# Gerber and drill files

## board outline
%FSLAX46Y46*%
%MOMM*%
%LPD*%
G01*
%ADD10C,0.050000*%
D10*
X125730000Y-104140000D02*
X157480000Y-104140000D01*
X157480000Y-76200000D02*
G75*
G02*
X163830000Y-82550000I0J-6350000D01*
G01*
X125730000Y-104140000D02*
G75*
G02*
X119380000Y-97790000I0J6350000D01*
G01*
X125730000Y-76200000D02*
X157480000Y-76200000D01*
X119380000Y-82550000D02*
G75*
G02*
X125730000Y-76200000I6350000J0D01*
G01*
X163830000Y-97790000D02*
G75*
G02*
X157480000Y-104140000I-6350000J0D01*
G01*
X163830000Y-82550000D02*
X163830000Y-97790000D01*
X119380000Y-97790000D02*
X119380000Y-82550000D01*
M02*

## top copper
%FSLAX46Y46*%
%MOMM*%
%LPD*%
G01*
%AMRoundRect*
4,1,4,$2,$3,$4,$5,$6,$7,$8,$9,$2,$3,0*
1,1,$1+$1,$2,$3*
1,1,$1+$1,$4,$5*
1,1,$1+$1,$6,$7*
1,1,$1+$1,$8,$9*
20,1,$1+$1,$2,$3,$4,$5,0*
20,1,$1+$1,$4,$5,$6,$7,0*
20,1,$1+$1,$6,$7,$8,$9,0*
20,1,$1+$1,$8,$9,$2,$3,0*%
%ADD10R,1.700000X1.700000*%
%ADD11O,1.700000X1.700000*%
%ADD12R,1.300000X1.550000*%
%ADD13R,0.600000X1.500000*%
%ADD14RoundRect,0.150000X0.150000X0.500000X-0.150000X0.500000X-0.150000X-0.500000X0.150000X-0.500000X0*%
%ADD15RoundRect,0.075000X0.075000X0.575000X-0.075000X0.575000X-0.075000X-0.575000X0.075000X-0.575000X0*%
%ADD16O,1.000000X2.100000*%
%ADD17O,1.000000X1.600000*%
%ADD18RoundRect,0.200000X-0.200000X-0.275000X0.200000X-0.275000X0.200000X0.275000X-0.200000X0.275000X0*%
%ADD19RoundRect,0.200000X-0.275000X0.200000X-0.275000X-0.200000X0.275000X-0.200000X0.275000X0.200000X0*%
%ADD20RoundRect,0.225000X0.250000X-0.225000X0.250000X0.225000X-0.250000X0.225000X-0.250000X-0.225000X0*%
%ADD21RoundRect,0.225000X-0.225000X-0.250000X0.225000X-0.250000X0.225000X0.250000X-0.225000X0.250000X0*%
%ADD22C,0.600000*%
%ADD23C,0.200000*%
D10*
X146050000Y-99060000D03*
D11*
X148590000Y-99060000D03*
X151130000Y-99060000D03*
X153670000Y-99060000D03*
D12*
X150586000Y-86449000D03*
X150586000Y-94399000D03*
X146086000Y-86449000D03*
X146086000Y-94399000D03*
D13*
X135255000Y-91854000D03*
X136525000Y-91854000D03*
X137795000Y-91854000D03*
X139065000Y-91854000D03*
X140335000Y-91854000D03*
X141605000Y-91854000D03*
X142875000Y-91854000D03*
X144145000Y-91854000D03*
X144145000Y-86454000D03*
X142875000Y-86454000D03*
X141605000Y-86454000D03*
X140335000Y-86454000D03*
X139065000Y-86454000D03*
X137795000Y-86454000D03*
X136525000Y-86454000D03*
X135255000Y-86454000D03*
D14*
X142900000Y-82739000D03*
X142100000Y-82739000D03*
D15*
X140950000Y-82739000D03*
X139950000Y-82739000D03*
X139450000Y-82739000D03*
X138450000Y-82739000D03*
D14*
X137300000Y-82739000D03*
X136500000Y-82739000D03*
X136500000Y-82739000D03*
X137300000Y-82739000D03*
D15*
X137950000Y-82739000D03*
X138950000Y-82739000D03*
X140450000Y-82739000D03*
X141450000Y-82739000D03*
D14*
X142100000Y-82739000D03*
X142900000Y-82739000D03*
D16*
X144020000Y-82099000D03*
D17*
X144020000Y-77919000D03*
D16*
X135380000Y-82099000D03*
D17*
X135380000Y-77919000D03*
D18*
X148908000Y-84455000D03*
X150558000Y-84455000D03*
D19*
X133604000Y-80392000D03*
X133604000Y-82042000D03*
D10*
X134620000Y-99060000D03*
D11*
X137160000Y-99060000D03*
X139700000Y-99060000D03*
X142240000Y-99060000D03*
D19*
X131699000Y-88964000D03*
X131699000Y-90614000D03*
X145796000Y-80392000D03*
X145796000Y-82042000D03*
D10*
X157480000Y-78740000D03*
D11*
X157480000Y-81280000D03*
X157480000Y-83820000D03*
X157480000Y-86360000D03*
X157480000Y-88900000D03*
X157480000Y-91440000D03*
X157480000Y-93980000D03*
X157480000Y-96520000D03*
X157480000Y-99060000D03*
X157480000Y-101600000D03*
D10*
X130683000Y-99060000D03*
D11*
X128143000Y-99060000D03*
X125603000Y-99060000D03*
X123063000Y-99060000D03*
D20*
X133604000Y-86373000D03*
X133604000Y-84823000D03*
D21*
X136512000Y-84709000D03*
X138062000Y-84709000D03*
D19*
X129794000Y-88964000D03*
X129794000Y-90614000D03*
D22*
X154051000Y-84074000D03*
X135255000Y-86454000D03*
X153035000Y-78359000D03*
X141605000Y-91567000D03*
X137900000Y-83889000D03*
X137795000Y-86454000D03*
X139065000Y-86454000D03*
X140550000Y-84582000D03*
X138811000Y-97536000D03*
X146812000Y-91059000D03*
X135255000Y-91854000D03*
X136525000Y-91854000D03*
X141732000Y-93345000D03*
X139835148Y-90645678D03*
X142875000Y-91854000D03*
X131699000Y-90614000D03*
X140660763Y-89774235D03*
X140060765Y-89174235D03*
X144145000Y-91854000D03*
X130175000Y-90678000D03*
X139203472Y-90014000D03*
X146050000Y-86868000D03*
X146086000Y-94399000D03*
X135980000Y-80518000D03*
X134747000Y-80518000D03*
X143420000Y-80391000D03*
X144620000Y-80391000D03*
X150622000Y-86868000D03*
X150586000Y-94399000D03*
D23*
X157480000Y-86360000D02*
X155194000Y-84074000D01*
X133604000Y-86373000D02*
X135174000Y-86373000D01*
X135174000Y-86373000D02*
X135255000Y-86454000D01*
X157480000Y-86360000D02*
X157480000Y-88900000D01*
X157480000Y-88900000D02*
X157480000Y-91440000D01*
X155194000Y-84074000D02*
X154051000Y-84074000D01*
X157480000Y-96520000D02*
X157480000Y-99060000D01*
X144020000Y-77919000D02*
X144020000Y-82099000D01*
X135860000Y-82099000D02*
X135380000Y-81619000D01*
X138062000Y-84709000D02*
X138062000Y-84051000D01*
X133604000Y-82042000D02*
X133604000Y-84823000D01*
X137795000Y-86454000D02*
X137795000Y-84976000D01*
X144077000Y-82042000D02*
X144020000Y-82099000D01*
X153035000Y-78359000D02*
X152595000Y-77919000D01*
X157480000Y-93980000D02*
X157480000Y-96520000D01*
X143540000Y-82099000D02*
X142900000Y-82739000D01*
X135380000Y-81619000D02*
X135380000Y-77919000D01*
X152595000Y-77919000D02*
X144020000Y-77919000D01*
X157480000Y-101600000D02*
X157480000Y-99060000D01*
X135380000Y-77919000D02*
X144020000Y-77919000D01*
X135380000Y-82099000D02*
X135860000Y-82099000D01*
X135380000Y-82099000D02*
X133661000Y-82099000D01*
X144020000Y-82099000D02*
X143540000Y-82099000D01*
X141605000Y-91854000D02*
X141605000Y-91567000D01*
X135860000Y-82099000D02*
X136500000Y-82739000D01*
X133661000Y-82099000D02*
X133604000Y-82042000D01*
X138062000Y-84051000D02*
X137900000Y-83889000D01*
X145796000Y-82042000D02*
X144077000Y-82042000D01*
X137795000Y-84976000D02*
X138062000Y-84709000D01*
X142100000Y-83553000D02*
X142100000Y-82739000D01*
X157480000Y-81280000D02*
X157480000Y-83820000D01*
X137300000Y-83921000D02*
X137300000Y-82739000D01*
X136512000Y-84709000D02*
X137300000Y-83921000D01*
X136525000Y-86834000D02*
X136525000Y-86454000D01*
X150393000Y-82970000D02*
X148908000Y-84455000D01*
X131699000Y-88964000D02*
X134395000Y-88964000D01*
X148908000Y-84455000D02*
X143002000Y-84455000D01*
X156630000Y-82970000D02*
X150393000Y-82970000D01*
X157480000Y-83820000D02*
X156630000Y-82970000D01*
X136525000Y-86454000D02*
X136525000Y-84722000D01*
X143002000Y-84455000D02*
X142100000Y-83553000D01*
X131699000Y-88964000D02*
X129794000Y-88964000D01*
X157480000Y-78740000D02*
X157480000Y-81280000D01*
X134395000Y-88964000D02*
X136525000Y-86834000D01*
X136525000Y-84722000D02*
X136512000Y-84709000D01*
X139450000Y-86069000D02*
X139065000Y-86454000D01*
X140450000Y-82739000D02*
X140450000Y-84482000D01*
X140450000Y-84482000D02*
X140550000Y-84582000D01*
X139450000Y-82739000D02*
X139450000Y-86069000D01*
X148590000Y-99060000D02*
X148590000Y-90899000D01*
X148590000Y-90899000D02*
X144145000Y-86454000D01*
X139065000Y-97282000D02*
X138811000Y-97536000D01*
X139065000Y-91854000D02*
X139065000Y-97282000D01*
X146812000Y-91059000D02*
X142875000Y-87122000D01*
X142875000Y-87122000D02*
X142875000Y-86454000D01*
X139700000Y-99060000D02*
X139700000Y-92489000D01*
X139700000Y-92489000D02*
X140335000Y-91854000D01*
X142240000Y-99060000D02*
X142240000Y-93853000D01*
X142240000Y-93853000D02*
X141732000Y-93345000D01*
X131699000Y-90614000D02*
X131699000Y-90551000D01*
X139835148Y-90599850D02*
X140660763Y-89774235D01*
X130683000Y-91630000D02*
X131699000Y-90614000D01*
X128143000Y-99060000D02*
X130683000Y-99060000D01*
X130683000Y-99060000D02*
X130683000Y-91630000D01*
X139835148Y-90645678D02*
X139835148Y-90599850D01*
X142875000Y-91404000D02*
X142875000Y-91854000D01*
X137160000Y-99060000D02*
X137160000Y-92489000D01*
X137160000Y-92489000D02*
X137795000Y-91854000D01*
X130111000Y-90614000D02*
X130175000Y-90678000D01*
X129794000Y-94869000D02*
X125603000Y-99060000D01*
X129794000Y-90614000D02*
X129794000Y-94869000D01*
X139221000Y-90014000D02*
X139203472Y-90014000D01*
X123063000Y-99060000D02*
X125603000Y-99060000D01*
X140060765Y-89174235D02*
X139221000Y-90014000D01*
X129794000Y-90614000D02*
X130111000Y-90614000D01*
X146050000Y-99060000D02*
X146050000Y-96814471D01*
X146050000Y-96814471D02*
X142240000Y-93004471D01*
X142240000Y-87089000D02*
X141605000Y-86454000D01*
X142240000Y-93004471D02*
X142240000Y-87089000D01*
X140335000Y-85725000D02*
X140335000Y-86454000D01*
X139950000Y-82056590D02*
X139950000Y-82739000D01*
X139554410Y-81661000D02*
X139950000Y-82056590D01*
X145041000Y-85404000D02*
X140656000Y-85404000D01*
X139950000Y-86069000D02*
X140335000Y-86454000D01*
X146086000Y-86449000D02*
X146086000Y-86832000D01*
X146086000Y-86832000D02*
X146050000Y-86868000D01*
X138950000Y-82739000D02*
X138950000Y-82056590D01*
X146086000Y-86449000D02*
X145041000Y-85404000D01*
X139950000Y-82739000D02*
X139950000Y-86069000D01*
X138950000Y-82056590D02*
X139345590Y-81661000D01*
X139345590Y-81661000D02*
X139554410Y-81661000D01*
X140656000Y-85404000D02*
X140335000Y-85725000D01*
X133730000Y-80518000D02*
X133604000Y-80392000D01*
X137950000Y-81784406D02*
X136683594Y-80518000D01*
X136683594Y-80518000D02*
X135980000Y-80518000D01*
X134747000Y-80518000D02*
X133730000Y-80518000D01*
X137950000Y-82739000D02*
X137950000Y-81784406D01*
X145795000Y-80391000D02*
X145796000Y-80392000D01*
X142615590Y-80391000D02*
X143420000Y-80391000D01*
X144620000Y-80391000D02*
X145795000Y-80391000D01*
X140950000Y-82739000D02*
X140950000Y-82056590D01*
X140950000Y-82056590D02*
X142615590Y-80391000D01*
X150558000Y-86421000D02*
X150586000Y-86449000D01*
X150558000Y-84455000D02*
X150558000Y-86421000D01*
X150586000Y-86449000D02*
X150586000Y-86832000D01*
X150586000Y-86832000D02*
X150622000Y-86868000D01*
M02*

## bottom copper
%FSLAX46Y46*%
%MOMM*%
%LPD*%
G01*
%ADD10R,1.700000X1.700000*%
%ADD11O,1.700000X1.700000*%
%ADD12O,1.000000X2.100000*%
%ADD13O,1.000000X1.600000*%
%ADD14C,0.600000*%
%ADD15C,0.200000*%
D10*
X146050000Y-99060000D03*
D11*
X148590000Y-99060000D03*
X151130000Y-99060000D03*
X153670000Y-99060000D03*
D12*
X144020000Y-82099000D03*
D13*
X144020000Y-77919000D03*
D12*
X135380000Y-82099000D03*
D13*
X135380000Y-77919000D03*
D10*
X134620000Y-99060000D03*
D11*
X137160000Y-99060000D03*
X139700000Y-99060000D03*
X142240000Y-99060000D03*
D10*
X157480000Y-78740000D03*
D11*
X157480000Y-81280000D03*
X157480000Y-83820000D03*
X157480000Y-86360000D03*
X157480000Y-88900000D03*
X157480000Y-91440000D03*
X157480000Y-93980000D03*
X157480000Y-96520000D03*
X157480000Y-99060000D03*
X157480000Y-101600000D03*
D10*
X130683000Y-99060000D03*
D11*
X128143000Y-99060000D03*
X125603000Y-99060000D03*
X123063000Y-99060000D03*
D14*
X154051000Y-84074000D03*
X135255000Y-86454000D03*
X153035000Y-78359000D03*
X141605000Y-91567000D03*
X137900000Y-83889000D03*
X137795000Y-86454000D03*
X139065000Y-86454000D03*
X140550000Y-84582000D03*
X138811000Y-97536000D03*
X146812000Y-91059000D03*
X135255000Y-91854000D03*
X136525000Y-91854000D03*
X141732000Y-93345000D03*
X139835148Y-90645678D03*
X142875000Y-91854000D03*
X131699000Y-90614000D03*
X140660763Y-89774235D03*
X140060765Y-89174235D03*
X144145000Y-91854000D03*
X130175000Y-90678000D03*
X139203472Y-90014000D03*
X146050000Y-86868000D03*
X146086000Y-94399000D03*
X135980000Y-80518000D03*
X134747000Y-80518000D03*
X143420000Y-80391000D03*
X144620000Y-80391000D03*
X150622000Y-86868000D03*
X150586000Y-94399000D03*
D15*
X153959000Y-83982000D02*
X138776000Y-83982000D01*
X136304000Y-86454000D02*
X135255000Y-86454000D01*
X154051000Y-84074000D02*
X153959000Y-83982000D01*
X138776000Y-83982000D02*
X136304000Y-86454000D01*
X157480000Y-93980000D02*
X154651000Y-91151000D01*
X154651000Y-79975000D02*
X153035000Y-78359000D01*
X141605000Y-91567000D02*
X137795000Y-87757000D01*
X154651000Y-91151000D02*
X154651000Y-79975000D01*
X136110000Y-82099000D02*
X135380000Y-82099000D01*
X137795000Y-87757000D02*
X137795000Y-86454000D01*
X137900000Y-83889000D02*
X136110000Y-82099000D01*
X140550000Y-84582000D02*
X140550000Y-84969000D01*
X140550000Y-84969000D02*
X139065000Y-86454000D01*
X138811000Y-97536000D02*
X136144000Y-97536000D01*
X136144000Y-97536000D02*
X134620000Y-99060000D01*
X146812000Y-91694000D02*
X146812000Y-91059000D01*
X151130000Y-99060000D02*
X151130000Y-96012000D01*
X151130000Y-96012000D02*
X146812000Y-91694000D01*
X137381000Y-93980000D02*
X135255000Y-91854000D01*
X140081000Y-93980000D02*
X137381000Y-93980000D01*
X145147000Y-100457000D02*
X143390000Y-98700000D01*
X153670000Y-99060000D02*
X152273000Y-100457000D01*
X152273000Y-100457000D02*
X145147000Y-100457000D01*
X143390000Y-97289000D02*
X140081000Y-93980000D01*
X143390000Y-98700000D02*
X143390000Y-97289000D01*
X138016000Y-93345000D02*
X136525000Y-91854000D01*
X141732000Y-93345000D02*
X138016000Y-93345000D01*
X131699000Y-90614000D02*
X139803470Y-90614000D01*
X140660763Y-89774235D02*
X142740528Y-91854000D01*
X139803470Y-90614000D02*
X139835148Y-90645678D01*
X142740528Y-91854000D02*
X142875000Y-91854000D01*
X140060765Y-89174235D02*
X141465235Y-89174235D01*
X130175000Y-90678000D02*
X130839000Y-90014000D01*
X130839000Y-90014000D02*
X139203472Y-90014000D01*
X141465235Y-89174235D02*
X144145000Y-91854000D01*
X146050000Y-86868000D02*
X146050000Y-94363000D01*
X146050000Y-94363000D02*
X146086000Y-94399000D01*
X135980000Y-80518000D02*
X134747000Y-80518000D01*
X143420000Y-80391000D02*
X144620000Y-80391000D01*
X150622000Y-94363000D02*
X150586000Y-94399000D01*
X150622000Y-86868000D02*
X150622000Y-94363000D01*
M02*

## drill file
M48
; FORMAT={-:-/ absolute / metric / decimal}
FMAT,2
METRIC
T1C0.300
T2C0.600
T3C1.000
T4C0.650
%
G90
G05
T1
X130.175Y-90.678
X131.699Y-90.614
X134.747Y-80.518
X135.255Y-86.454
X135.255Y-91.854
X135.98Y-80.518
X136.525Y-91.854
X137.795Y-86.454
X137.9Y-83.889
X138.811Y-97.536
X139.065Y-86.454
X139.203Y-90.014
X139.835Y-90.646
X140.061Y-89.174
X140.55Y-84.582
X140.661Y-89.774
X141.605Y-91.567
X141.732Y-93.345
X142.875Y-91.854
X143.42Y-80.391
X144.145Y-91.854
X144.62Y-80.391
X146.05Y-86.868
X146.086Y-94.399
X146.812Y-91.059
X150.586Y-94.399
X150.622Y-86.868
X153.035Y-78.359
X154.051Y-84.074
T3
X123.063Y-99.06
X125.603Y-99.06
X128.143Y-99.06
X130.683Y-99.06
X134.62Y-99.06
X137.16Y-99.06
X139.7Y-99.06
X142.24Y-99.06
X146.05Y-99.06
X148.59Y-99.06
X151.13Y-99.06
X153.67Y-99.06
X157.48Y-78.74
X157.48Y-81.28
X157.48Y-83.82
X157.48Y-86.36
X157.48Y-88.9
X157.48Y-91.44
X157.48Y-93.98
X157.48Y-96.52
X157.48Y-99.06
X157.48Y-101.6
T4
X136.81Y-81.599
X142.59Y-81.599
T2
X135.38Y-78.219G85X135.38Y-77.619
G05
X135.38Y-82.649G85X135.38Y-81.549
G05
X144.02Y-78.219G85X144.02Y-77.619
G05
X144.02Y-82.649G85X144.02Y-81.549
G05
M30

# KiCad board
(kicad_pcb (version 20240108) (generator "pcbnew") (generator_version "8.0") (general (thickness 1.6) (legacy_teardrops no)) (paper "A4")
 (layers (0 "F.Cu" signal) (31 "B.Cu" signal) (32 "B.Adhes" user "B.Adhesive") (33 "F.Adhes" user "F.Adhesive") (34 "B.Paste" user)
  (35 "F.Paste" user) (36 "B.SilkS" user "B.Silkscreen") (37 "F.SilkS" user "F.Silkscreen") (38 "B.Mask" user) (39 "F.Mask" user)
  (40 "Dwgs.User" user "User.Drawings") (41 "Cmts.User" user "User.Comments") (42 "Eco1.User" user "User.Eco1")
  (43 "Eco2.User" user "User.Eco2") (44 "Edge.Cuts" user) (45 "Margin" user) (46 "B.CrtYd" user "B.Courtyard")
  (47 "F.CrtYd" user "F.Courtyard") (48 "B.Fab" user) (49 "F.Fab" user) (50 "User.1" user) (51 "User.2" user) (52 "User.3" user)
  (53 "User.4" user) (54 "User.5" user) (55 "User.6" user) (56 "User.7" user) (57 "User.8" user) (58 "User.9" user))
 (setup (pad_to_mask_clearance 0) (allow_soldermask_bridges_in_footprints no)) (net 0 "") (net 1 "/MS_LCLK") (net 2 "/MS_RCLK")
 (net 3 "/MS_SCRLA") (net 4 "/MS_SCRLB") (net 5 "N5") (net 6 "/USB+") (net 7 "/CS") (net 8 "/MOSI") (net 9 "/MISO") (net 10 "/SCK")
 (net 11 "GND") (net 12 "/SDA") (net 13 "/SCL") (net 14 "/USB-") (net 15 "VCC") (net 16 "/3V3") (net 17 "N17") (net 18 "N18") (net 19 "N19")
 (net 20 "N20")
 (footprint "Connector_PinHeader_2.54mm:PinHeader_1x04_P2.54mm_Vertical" (layer "F.Cu") (at 146.05 99.06 90)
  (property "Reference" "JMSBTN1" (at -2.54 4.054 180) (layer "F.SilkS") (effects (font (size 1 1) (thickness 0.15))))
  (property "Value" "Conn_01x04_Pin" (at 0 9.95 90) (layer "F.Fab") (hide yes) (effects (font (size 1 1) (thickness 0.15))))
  (pad "1" thru_hole rect (at 0 0 90) (size 1.7 1.7) (drill 1) (layers "*.Cu" "*.Mask") (remove_unused_layers no) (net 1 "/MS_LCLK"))
  (pad "2" thru_hole oval (at 0 2.54 90) (size 1.7 1.7) (drill 1) (layers "*.Cu" "*.Mask") (remove_unused_layers no) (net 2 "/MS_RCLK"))
  (pad "3" thru_hole oval (at 0 5.08 90) (size 1.7 1.7) (drill 1) (layers "*.Cu" "*.Mask") (remove_unused_layers no) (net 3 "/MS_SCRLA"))
  (pad "4" thru_hole oval (at 0 7.62 90) (size 1.7 1.7) (drill 1) (layers "*.Cu" "*.Mask") (remove_unused_layers no) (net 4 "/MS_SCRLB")))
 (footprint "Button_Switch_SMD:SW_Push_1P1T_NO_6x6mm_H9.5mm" (layer "F.Cu") (at 148.336 90.424 -90)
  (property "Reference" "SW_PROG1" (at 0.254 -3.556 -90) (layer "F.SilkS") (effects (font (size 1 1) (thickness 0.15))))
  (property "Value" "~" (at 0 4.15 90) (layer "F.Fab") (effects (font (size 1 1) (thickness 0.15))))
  (pad "1" smd rect (at -3.975 -2.25 270) (size 1.55 1.3) (layers "F.Cu" "F.Paste" "F.Mask") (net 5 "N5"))
  (pad "1" smd rect (at 3.975 -2.25 270) (size 1.55 1.3) (layers "F.Cu" "F.Paste" "F.Mask") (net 5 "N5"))
  (pad "2" smd rect (at -3.975 2.25 270) (size 1.55 1.3) (layers "F.Cu" "F.Paste" "F.Mask") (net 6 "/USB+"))
  (pad "2" smd rect (at 3.975 2.25 270) (size 1.55 1.3) (layers "F.Cu" "F.Paste" "F.Mask") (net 6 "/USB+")))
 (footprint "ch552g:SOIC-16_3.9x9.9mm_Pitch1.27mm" (layer "F.Cu") (at 139.7 89.154 90)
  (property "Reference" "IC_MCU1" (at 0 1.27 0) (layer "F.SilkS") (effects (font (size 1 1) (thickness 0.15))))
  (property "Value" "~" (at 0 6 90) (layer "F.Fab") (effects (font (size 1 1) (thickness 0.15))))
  (pad "1" smd rect (at -2.7 -4.445 90) (size 1.5 0.6) (layers "F.Cu" "F.Paste" "F.Mask") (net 4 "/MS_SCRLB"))
  (pad "2" smd rect (at -2.7 -3.175 90) (size 1.5 0.6) (layers "F.Cu" "F.Paste" "F.Mask") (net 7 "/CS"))
  (pad "3" smd rect (at -2.7 -1.905 90) (size 1.5 0.6) (layers "F.Cu" "F.Paste" "F.Mask") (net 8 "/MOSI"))
  (pad "4" smd rect (at -2.7 -0.635 90) (size 1.5 0.6) (layers "F.Cu" "F.Paste" "F.Mask") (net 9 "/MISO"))
  (pad "5" smd rect (at -2.7 0.635 90) (size 1.5 0.6) (layers "F.Cu" "F.Paste" "F.Mask") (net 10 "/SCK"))
  (pad "6" smd rect (at -2.7 1.905 90) (size 1.5 0.6) (layers "F.Cu" "F.Paste" "F.Mask") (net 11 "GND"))
  (pad "7" smd rect (at -2.7 3.175 90) (size 1.5 0.6) (layers "F.Cu" "F.Paste" "F.Mask") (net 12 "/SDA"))
  (pad "8" smd rect (at -2.7 4.445 90) (size 1.5 0.6) (layers "F.Cu" "F.Paste" "F.Mask") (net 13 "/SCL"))
  (pad "9" smd rect (at 2.7 4.445 90) (size 1.5 0.6) (layers "F.Cu" "F.Paste" "F.Mask") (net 2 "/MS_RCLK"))
  (pad "10" smd rect (at 2.7 3.175 90) (size 1.5 0.6) (layers "F.Cu" "F.Paste" "F.Mask") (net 3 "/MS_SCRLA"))
  (pad "11" smd rect (at 2.7 1.905 90) (size 1.5 0.6) (layers "F.Cu" "F.Paste" "F.Mask") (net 1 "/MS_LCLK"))
  (pad "12" smd rect (at 2.7 0.635 90) (size 1.5 0.6) (layers "F.Cu" "F.Paste" "F.Mask") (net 6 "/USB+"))
  (pad "13" smd rect (at 2.7 -0.635 90) (size 1.5 0.6) (layers "F.Cu" "F.Paste" "F.Mask") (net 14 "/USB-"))
  (pad "14" smd rect (at 2.7 -1.905 90) (size 1.5 0.6) (layers "F.Cu" "F.Paste" "F.Mask") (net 11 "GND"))
  (pad "15" smd rect (at 2.7 -3.175 90) (size 1.5 0.6) (layers "F.Cu" "F.Paste" "F.Mask") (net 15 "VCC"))
  (pad "16" smd rect (at 2.7 -4.445 90) (size 1.5 0.6) (layers "F.Cu" "F.Paste" "F.Mask") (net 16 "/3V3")))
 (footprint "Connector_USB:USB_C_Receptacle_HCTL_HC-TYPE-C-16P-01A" (layer "F.Cu") (at 139.7 78.994 180)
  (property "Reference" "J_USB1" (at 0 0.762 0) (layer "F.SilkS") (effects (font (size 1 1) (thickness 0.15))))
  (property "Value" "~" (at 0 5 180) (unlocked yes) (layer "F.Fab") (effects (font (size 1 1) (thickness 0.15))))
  (pad "" np_thru_hole circle (at -2.89 -2.605 180) (size 0.65 0.65) (drill 0.65) (layers "*.Mask"))
  (pad "" np_thru_hole circle (at 2.89 -2.605 180) (size 0.65 0.65) (drill 0.65) (layers "*.Mask"))
  (pad "A1" smd roundrect (at -3.2 -3.745 180) (size 0.6 1.3) (layers "F.Cu" "F.Paste" "F.Mask") (roundrect_rratio 0.25) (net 11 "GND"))
  (pad "A4" smd roundrect (at -2.4 -3.745 180) (size 0.6 1.3) (layers "F.Cu" "F.Paste" "F.Mask") (roundrect_rratio 0.25) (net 15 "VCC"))
  (pad "A5" smd roundrect (at -1.25 -3.745 180) (size 0.3 1.3) (layers "F.Cu" "F.Paste" "F.Mask") (roundrect_rratio 0.25) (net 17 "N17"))
  (pad "A6" smd roundrect (at -0.25 -3.745 180) (size 0.3 1.3) (layers "F.Cu" "F.Paste" "F.Mask") (roundrect_rratio 0.25) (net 6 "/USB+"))
  (pad "A7" smd roundrect (at 0.25 -3.745 180) (size 0.3 1.3) (layers "F.Cu" "F.Paste" "F.Mask") (roundrect_rratio 0.25) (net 14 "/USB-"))
  (pad "A8" smd roundrect (at 1.25 -3.745 180) (size 0.3 1.3) (layers "F.Cu" "F.Paste" "F.Mask") (roundrect_rratio 0.25) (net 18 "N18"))
  (pad "A9" smd roundrect (at 2.4 -3.745 180) (size 0.6 1.3) (layers "F.Cu" "F.Paste" "F.Mask") (roundrect_rratio 0.25) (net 15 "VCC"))
  (pad "A12" smd roundrect (at 3.2 -3.745 180) (size 0.6 1.3) (layers "F.Cu" "F.Paste" "F.Mask") (roundrect_rratio 0.25) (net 11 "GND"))
  (pad "B1" smd roundrect (at 3.2 -3.745 180) (size 0.6 1.3) (layers "F.Cu" "F.Paste" "F.Mask") (roundrect_rratio 0.25) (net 11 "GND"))
  (pad "B4" smd roundrect (at 2.4 -3.745 180) (size 0.6 1.3) (layers "F.Cu" "F.Paste" "F.Mask") (roundrect_rratio 0.25) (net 15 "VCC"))
  (pad "B5" smd roundrect (at 1.75 -3.745 180) (size 0.3 1.3) (layers "F.Cu" "F.Paste" "F.Mask") (roundrect_rratio 0.25) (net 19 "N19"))
  (pad "B6" smd roundrect (at 0.75 -3.745 180) (size 0.3 1.3) (layers "F.Cu" "F.Paste" "F.Mask") (roundrect_rratio 0.25) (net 6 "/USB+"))
  (pad "B7" smd roundrect (at -0.75 -3.745 180) (size 0.3 1.3) (layers "F.Cu" "F.Paste" "F.Mask") (roundrect_rratio 0.25) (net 14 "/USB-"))
  (pad "B8" smd roundrect (at -1.75 -3.745 180) (size 0.3 1.3) (layers "F.Cu" "F.Paste" "F.Mask") (roundrect_rratio 0.25) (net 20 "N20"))
  (pad "B9" smd roundrect (at -2.4 -3.745 180) (size 0.6 1.3) (layers "F.Cu" "F.Paste" "F.Mask") (roundrect_rratio 0.25) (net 15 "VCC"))
  (pad "B12" smd roundrect (at -3.2 -3.745 180) (size 0.6 1.3) (layers "F.Cu" "F.Paste" "F.Mask") (roundrect_rratio 0.25) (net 11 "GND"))
  (pad "S1" thru_hole oval (at -4.32 -3.105 180) (size 1 2.1) (drill oval 0.6 1.7) (layers "*.Cu" "*.Mask") (remove_unused_layers no)
   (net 11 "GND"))
  (pad "S1" thru_hole oval (at -4.32 1.075 180) (size 1 1.6) (drill oval 0.6 1.2) (layers "*.Cu" "*.Mask") (remove_unused_layers no)
   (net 11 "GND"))
  (pad "S1" thru_hole oval (at 4.32 -3.105 180) (size 1 2.1) (drill oval 0.6 1.7) (layers "*.Cu" "*.Mask") (remove_unused_layers no)
   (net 11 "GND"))
  (pad "S1" thru_hole oval (at 4.32 1.075 180) (size 1 1.6) (drill oval 0.6 1.2) (layers "*.Cu" "*.Mask") (remove_unused_layers no)
   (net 11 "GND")))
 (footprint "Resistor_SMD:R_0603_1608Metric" (layer "F.Cu") (at 149.733 84.455)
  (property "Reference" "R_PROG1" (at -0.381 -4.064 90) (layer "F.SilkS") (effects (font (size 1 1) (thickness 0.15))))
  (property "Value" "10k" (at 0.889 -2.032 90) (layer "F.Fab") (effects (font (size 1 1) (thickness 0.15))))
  (pad "1" smd roundrect (at -0.825 0) (size 0.8 0.95) (layers "F.Cu" "F.Paste" "F.Mask") (roundrect_rratio 0.25) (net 15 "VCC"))
  (pad "2" smd roundrect (at 0.825 0) (size 0.8 0.95) (layers "F.Cu" "F.Paste" "F.Mask") (roundrect_rratio 0.25) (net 5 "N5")))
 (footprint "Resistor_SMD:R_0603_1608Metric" (layer "F.Cu") (at 133.604 81.217 -90)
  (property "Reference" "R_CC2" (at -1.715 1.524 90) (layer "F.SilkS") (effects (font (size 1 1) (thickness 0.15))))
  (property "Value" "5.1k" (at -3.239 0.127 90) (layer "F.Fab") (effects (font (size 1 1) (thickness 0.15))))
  (pad "1" smd roundrect (at -0.825 0 270) (size 0.8 0.95) (layers "F.Cu" "F.Paste" "F.Mask") (roundrect_rratio 0.25) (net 19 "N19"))
  (pad "2" smd roundrect (at 0.825 0 270) (size 0.8 0.95) (layers "F.Cu" "F.Paste" "F.Mask") (roundrect_rratio 0.25) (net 11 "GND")))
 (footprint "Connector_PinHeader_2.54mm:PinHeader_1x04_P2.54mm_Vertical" (layer "F.Cu") (at 134.62 99.06 90)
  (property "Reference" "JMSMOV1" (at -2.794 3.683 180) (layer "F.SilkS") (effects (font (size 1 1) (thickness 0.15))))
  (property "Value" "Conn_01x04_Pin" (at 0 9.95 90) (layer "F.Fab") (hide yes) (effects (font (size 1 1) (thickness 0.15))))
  (pad "1" thru_hole rect (at 0 0 90) (size 1.7 1.7) (drill 1) (layers "*.Cu" "*.Mask") (remove_unused_layers no) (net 9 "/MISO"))
  (pad "2" thru_hole oval (at 0 2.54 90) (size 1.7 1.7) (drill 1) (layers "*.Cu" "*.Mask") (remove_unused_layers no) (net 8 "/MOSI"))
  (pad "3" thru_hole oval (at 0 5.08 90) (size 1.7 1.7) (drill 1) (layers "*.Cu" "*.Mask") (remove_unused_layers no) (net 10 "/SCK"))
  (pad "4" thru_hole oval (at 0 7.62 90) (size 1.7 1.7) (drill 1) (layers "*.Cu" "*.Mask") (remove_unused_layers no) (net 7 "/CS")))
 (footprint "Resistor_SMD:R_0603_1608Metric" (layer "F.Cu") (at 131.699 89.789 -90)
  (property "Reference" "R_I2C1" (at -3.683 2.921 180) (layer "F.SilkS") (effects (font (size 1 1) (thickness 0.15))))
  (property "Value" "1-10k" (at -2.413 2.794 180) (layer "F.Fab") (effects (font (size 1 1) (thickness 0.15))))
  (pad "1" smd roundrect (at -0.825 0 270) (size 0.8 0.95) (layers "F.Cu" "F.Paste" "F.Mask") (roundrect_rratio 0.25) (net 15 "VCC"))
  (pad "2" smd roundrect (at 0.825 0 270) (size 0.8 0.95) (layers "F.Cu" "F.Paste" "F.Mask") (roundrect_rratio 0.25) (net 12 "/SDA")))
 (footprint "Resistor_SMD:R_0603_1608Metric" (layer "F.Cu") (at 145.796 81.217 -90)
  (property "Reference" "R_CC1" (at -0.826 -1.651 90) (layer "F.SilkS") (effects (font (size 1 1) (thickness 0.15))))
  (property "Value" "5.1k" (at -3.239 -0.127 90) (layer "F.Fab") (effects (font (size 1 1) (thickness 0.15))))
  (pad "1" smd roundrect (at -0.825 0 270) (size 0.8 0.95) (layers "F.Cu" "F.Paste" "F.Mask") (roundrect_rratio 0.25) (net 17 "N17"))
  (pad "2" smd roundrect (at 0.825 0 270) (size 0.8 0.95) (layers "F.Cu" "F.Paste" "F.Mask") (roundrect_rratio 0.25) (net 11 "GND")))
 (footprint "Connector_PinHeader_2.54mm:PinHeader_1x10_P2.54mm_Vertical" (layer "F.Cu") (at 157.48 78.74)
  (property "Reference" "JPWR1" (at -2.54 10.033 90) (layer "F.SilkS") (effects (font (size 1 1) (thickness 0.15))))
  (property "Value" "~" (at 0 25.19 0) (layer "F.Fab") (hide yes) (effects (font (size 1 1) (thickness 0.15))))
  (pad "1" thru_hole rect (at 0 0) (size 1.7 1.7) (drill 1) (layers "*.Cu" "*.Mask") (remove_unused_layers no) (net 15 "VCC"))
  (pad "2" thru_hole oval (at 0 2.54) (size 1.7 1.7) (drill 1) (layers "*.Cu" "*.Mask") (remove_unused_layers no) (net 15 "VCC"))
  (pad "3" thru_hole oval (at 0 5.08) (size 1.7 1.7) (drill 1) (layers "*.Cu" "*.Mask") (remove_unused_layers no) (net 15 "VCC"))
  (pad "4" thru_hole oval (at 0 7.62) (size 1.7 1.7) (drill 1) (layers "*.Cu" "*.Mask") (remove_unused_layers no) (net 16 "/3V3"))
  (pad "5" thru_hole oval (at 0 10.16) (size 1.7 1.7) (drill 1) (layers "*.Cu" "*.Mask") (remove_unused_layers no) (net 16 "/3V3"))
  (pad "6" thru_hole oval (at 0 12.7) (size 1.7 1.7) (drill 1) (layers "*.Cu" "*.Mask") (remove_unused_layers no) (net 16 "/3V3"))
  (pad "7" thru_hole oval (at 0 15.24) (size 1.7 1.7) (drill 1) (layers "*.Cu" "*.Mask") (remove_unused_layers no) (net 11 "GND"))
  (pad "8" thru_hole oval (at 0 17.78) (size 1.7 1.7) (drill 1) (layers "*.Cu" "*.Mask") (remove_unused_layers no) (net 11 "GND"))
  (pad "9" thru_hole oval (at 0 20.32) (size 1.7 1.7) (drill 1) (layers "*.Cu" "*.Mask") (remove_unused_layers no) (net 11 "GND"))
  (pad "10" thru_hole oval (at 0 22.86) (size 1.7 1.7) (drill 1) (layers "*.Cu" "*.Mask") (remove_unused_layers no) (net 11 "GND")))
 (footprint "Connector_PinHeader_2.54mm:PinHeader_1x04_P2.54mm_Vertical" (layer "F.Cu") (at 130.683 99.06 -90)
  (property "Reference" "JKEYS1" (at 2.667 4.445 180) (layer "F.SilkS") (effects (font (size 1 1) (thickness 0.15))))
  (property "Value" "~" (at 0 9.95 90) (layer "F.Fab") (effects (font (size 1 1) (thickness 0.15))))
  (pad "1" thru_hole rect (at 0 0 270) (size 1.7 1.7) (drill 1) (layers "*.Cu" "*.Mask") (remove_unused_layers no) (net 12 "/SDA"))
  (pad "2" thru_hole oval (at 0 2.54 270) (size 1.7 1.7) (drill 1) (layers "*.Cu" "*.Mask") (remove_unused_layers no) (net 12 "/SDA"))
  (pad "3" thru_hole oval (at 0 5.08 270) (size 1.7 1.7) (drill 1) (layers "*.Cu" "*.Mask") (remove_unused_layers no) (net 13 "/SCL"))
  (pad "4" thru_hole oval (at 0 7.62 270) (size 1.7 1.7) (drill 1) (layers "*.Cu" "*.Mask") (remove_unused_layers no) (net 13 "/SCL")))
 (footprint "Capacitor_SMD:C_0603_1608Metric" (layer "F.Cu") (at 133.604 85.598 90)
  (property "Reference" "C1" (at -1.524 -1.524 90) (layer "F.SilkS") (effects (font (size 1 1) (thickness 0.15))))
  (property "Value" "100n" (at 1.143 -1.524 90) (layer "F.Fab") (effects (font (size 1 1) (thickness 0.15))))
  (pad "1" smd roundrect (at -0.775 0 90) (size 0.9 0.95) (layers "F.Cu" "F.Paste" "F.Mask") (roundrect_rratio 0.25) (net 16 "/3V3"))
  (pad "2" smd roundrect (at 0.775 0 90) (size 0.9 0.95) (layers "F.Cu" "F.Paste" "F.Mask") (roundrect_rratio 0.25) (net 11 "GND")))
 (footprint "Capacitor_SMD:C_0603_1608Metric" (layer "F.Cu") (at 137.287 84.709)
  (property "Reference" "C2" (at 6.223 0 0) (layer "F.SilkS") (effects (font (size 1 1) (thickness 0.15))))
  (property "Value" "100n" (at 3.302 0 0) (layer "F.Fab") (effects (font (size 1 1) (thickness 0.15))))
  (pad "1" smd roundrect (at -0.775 0) (size 0.9 0.95) (layers "F.Cu" "F.Paste" "F.Mask") (roundrect_rratio 0.25) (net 15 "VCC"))
  (pad "2" smd roundrect (at 0.775 0) (size 0.9 0.95) (layers "F.Cu" "F.Paste" "F.Mask") (roundrect_rratio 0.25) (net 11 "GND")))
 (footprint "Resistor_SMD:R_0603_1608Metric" (layer "F.Cu") (at 129.794 89.789 -90)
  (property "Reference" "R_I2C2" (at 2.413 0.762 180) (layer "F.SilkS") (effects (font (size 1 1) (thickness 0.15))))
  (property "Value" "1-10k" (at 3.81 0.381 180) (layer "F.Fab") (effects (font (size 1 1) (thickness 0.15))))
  (pad "1" smd roundrect (at -0.825 0 270) (size 0.8 0.95) (layers "F.Cu" "F.Paste" "F.Mask") (roundrect_rratio 0.25) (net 15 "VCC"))
  (pad "2" smd roundrect (at 0.825 0 270) (size 0.8 0.95) (layers "F.Cu" "F.Paste" "F.Mask") (roundrect_rratio 0.25) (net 13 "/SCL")))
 (gr_line (start 125.73 104.14) (end 157.48 104.14) (stroke (width 0.05) (type default)) (layer "Edge.Cuts"))
 (gr_arc (start 157.48 76.2) (mid 161.970128 78.059872) (end 163.83 82.55) (stroke (width 0.05) (type default)) (layer "Edge.Cuts"))
 (gr_arc (start 125.73 104.14) (mid 121.239872 102.280128) (end 119.38 97.79) (stroke (width 0.05) (type default)) (layer "Edge.Cuts"))
 (gr_line (start 125.73 76.2) (end 157.48 76.2) (stroke (width 0.05) (type default)) (layer "Edge.Cuts"))
 (gr_arc (start 119.38 82.55) (mid 121.239872 78.059872) (end 125.73 76.2) (stroke (width 0.05) (type default)) (layer "Edge.Cuts"))
 (gr_arc (start 163.83 97.79) (mid 161.970128 102.280128) (end 157.48 104.14) (stroke (width 0.05) (type default)) (layer "Edge.Cuts"))
 (gr_line (start 163.83 82.55) (end 163.83 97.79) (stroke (width 0.05) (type default)) (layer "Edge.Cuts"))
 (gr_line (start 119.38 97.79) (end 119.38 82.55) (stroke (width 0.05) (type default)) (layer "Edge.Cuts"))
 (segment (start 157.48 86.36) (end 155.194 84.074) (width 0.2) (layer "F.Cu") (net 16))
 (segment (start 133.604 86.373) (end 135.174 86.373) (width 0.2) (layer "F.Cu") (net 16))
 (segment (start 135.174 86.373) (end 135.255 86.454) (width 0.2) (layer "F.Cu") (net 16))
 (segment (start 157.48 86.36) (end 157.48 88.9) (width 0.2) (layer "F.Cu") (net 16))
 (segment (start 157.48 88.9) (end 157.48 91.44) (width 0.2) (layer "F.Cu") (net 16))
 (segment (start 155.194 84.074) (end 154.051 84.074) (width 0.2) (layer "F.Cu") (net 16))
 (via (at 154.051 84.074) (size 0.6) (drill 0.3) (layers "F.Cu" "B.Cu") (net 16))
 (via (at 135.255 86.454) (size 0.6) (drill 0.3) (layers "F.Cu" "B.Cu") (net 16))
 (segment (start 153.959 83.982) (end 138.776 83.982) (width 0.2) (layer "B.Cu") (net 16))
 (segment (start 136.304 86.454) (end 135.255 86.454) (width 0.2) (layer "B.Cu") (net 16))
 (segment (start 154.051 84.074) (end 153.959 83.982) (width 0.2) (layer "B.Cu") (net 16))
 (segment (start 138.776 83.982) (end 136.304 86.454) (width 0.2) (layer "B.Cu") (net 16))
 (segment (start 157.48 96.52) (end 157.48 99.06) (width 0.2) (layer "F.Cu") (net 11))
 (segment (start 144.02 77.919) (end 144.02 82.099) (width 0.2) (layer "F.Cu") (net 11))
 (segment (start 135.86 82.099) (end 135.38 81.619) (width 0.2) (layer "F.Cu") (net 11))
 (segment (start 138.062 84.709) (end 138.062 84.051) (width 0.2) (layer "F.Cu") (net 11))
 (segment (start 133.604 82.042) (end 133.604 84.823) (width 0.2) (layer "F.Cu") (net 11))
 (segment (start 137.795 86.454) (end 137.795 84.976) (width 0.2) (layer "F.Cu") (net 11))
 (segment (start 144.077 82.042) (end 144.02 82.099) (width 0.2) (layer "F.Cu") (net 11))
 (segment (start 153.035 78.359) (end 152.595 77.919) (width 0.2) (layer "F.Cu") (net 11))
 (segment (start 157.48 93.98) (end 157.48 96.52) (width 0.2) (layer "F.Cu") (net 11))
 (segment (start 143.54 82.099) (end 142.9 82.739) (width 0.2) (layer "F.Cu") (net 11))
 (segment (start 135.38 81.619) (end 135.38 77.919) (width 0.2) (layer "F.Cu") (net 11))
 (segment (start 152.595 77.919) (end 144.02 77.919) (width 0.2) (layer "F.Cu") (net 11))
 (segment (start 157.48 101.6) (end 157.48 99.06) (width 0.2) (layer "F.Cu") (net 11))
 (segment (start 135.38 77.919) (end 144.02 77.919) (width 0.2) (layer "F.Cu") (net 11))
 (segment (start 135.38 82.099) (end 135.86 82.099) (width 0.2) (layer "F.Cu") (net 11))
 (segment (start 135.38 82.099) (end 133.661 82.099) (width 0.2) (layer "F.Cu") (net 11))
 (segment (start 144.02 82.099) (end 143.54 82.099) (width 0.2) (layer "F.Cu") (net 11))
 (segment (start 141.605 91.854) (end 141.605 91.567) (width 0.2) (layer "F.Cu") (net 11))
 (segment (start 135.86 82.099) (end 136.5 82.739) (width 0.2) (layer "F.Cu") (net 11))
 (segment (start 133.661 82.099) (end 133.604 82.042) (width 0.2) (layer "F.Cu") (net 11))
 (segment (start 138.062 84.051) (end 137.9 83.889) (width 0.2) (layer "F.Cu") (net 11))
 (segment (start 145.796 82.042) (end 144.077 82.042) (width 0.2) (layer "F.Cu") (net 11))
 (segment (start 137.795 84.976) (end 138.062 84.709) (width 0.2) (layer "F.Cu") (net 11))
 (via (at 153.035 78.359) (size 0.6) (drill 0.3) (layers "F.Cu" "B.Cu") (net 11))
 (via (at 141.605 91.567) (size 0.6) (drill 0.3) (layers "F.Cu" "B.Cu") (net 11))
 (via (at 137.9 83.889) (size 0.6) (drill 0.3) (layers "F.Cu" "B.Cu") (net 11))
 (via (at 137.795 86.454) (size 0.6) (drill 0.3) (layers "F.Cu" "B.Cu") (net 11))
 (segment (start 157.48 93.98) (end 154.651 91.151) (width 0.2) (layer "B.Cu") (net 11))
 (segment (start 154.651 79.975) (end 153.035 78.359) (width 0.2) (layer "B.Cu") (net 11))
 (segment (start 141.605 91.567) (end 137.795 87.757) (width 0.2) (layer "B.Cu") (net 11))
 (segment (start 154.651 91.151) (end 154.651 79.975) (width 0.2) (layer "B.Cu") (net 11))
 (segment (start 136.11 82.099) (end 135.38 82.099) (width 0.2) (layer "B.Cu") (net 11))
 (segment (start 137.795 87.757) (end 137.795 86.454) (width 0.2) (layer "B.Cu") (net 11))
 (segment (start 137.9 83.889) (end 136.11 82.099) (width 0.2) (layer "B.Cu") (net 11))
 (segment (start 142.1 83.553) (end 142.1 82.739) (width 0.2) (layer "F.Cu") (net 15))
 (segment (start 157.48 81.28) (end 157.48 83.82) (width 0.2) (layer "F.Cu") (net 15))
 (segment (start 137.3 83.921) (end 137.3 82.739) (width 0.2) (layer "F.Cu") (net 15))
 (segment (start 136.512 84.709) (end 137.3 83.921) (width 0.2) (layer "F.Cu") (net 15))
 (segment (start 136.525 86.834) (end 136.525 86.454) (width 0.2) (layer "F.Cu") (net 15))
 (segment (start 150.393 82.97) (end 148.908 84.455) (width 0.2) (layer "F.Cu") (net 15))
 (segment (start 131.699 88.964) (end 134.395 88.964) (width 0.2) (layer "F.Cu") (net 15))
 (segment (start 148.908 84.455) (end 143.002 84.455) (width 0.2) (layer "F.Cu") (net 15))
 (segment (start 156.63 82.97) (end 150.393 82.97) (width 0.2) (layer "F.Cu") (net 15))
 (segment (start 157.48 83.82) (end 156.63 82.97) (width 0.2) (layer "F.Cu") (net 15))
 (segment (start 136.525 86.454) (end 136.525 84.722) (width 0.2) (layer "F.Cu") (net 15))
 (segment (start 143.002 84.455) (end 142.1 83.553) (width 0.2) (layer "F.Cu") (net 15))
 (segment (start 131.699 88.964) (end 129.794 88.964) (width 0.2) (layer "F.Cu") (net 15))
 (segment (start 157.48 78.74) (end 157.48 81.28) (width 0.2) (layer "F.Cu") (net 15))
 (segment (start 134.395 88.964) (end 136.525 86.834) (width 0.2) (layer "F.Cu") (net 15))
 (segment (start 136.525 84.722) (end 136.512 84.709) (width 0.2) (layer "F.Cu") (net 15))
 (segment (start 139.45 86.069) (end 139.065 86.454) (width 0.2) (layer "F.Cu") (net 14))
 (segment (start 140.45 82.739) (end 140.45 84.482) (width 0.2) (layer "F.Cu") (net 14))
 (segment (start 140.45 84.482) (end 140.55 84.582) (width 0.2) (layer "F.Cu") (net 14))
 (segment (start 139.45 82.739) (end 139.45 86.069) (width 0.2) (layer "F.Cu") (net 14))
 (via (at 139.065 86.454) (size 0.6) (drill 0.3) (layers "F.Cu" "B.Cu") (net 14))
 (via (at 140.55 84.582) (size 0.6) (drill 0.3) (layers "F.Cu" "B.Cu") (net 14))
 (segment (start 140.55 84.582) (end 140.55 84.969) (width 0.2) (layer "B.Cu") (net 14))
 (segment (start 140.55 84.969) (end 139.065 86.454) (width 0.2) (layer "B.Cu") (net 14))
 (segment (start 148.59 99.06) (end 148.59 90.899) (width 0.2) (layer "F.Cu") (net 2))
 (segment (start 148.59 90.899) (end 144.145 86.454) (width 0.2) (layer "F.Cu") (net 2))
 (segment (start 139.065 97.282) (end 138.811 97.536) (width 0.2) (layer "F.Cu") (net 9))
 (segment (start 139.065 91.854) (end 139.065 97.282) (width 0.2) (layer "F.Cu") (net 9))
 (via (at 138.811 97.536) (size 0.6) (drill 0.3) (layers "F.Cu" "B.Cu") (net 9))
 (segment (start 138.811 97.536) (end 136.144 97.536) (width 0.2) (layer "B.Cu") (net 9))
 (segment (start 136.144 97.536) (end 134.62 99.06) (width 0.2) (layer "B.Cu") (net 9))
 (segment (start 146.812 91.059) (end 142.875 87.122) (width 0.2) (layer "F.Cu") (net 3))
 (segment (start 142.875 87.122) (end 142.875 86.454) (width 0.2) (layer "F.Cu") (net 3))
 (via (at 146.812 91.059) (size 0.6) (drill 0.3) (layers "F.Cu" "B.Cu") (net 3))
 (segment (start 146.812 91.694) (end 146.812 91.059) (width 0.2) (layer "B.Cu") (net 3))
 (segment (start 151.13 99.06) (end 151.13 96.012) (width 0.2) (layer "B.Cu") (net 3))
 (segment (start 151.13 96.012) (end 146.812 91.694) (width 0.2) (layer "B.Cu") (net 3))
 (via (at 135.255 91.854) (size 0.6) (drill 0.3) (layers "F.Cu" "B.Cu") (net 4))
 (segment (start 137.381 93.98) (end 135.255 91.854) (width 0.2) (layer "B.Cu") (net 4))
 (segment (start 140.081 93.98) (end 137.381 93.98) (width 0.2) (layer "B.Cu") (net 4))
 (segment (start 145.147 100.457) (end 143.39 98.7) (width 0.2) (layer "B.Cu") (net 4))
 (segment (start 153.67 99.06) (end 152.273 100.457) (width 0.2) (layer "B.Cu") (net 4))
 (segment (start 152.273 100.457) (end 145.147 100.457) (width 0.2) (layer "B.Cu") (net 4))
 (segment (start 143.39 97.289) (end 140.081 93.98) (width 0.2) (layer "B.Cu") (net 4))
 (segment (start 143.39 98.7) (end 143.39 97.289) (width 0.2) (layer "B.Cu") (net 4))
 (segment (start 139.7 99.06) (end 139.7 92.489) (width 0.2) (layer "F.Cu") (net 10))
 (segment (start 139.7 92.489) (end 140.335 91.854) (width 0.2) (layer "F.Cu") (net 10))
 (segment (start 142.24 99.06) (end 142.24 93.853) (width 0.2) (layer "F.Cu") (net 7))
 (segment (start 142.24 93.853) (end 141.732 93.345) (width 0.2) (layer "F.Cu") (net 7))
 (via (at 136.525 91.854) (size 0.6) (drill 0.3) (layers "F.Cu" "B.Cu") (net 7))
 (via (at 141.732 93.345) (size 0.6) (drill 0.3) (layers "F.Cu" "B.Cu") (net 7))
 (segment (start 138.016 93.345) (end 136.525 91.854) (width 0.2) (layer "B.Cu") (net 7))
 (segment (start 141.732 93.345) (end 138.016 93.345) (width 0.2) (layer "B.Cu") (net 7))
 (segment (start 131.699 90.614) (end 131.699 90.551) (width 0.2) (layer "F.Cu") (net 12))
 (segment (start 139.835148 90.59985) (end 140.660763 89.774235) (width 0.2) (layer "F.Cu") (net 12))
 (segment (start 130.683 91.63) (end 131.699 90.614) (width 0.2) (layer "F.Cu") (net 12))
 (segment (start 128.143 99.06) (end 130.683 99.06) (width 0.2) (layer "F.Cu") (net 12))
 (segment (start 130.683 99.06) (end 130.683 91.63) (width 0.2) (layer "F.Cu") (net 12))
 (segment (start 139.835148 90.645678) (end 139.835148 90.59985) (width 0.2) (layer "F.Cu") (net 12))
 (segment (start 142.875 91.404) (end 142.875 91.854) (width 0.2) (layer "F.Cu") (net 12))
 (via (at 139.835148 90.645678) (size 0.6) (drill 0.3) (layers "F.Cu" "B.Cu") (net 12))
 (via (at 142.875 91.854) (size 0.6) (drill 0.3) (layers "F.Cu" "B.Cu") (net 12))
 (via (at 131.699 90.614) (size 0.6) (drill 0.3) (layers "F.Cu" "B.Cu") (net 12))
 (via (at 140.660763 89.774235) (size 0.6) (drill 0.3) (layers "F.Cu" "B.Cu") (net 12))
 (segment (start 131.699 90.614) (end 139.80347 90.614) (width 0.2) (layer "B.Cu") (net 12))
 (segment (start 140.660763 89.774235) (end 142.740528 91.854) (width 0.2) (layer "B.Cu") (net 12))
 (segment (start 139.80347 90.614) (end 139.835148 90.645678) (width 0.2) (layer "B.Cu") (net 12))
 (segment (start 142.740528 91.854) (end 142.875 91.854) (width 0.2) (layer "B.Cu") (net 12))
 (segment (start 137.16 99.06) (end 137.16 92.489) (width 0.2) (layer "F.Cu") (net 8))
 (segment (start 137.16 92.489) (end 137.795 91.854) (width 0.2) (layer "F.Cu") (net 8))
 (segment (start 130.111 90.614) (end 130.175 90.678) (width 0.2) (layer "F.Cu") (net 13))
 (segment (start 129.794 94.869) (end 125.603 99.06) (width 0.2) (layer "F.Cu") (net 13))
 (segment (start 129.794 90.614) (end 129.794 94.869) (width 0.2) (layer "F.Cu") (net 13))
 (segment (start 139.221 90.014) (end 139.203472 90.014) (width 0.2) (layer "F.Cu") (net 13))
 (segment (start 123.063 99.06) (end 125.603 99.06) (width 0.2) (layer "F.Cu") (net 13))
 (segment (start 140.060765 89.174235) (end 139.221 90.014) (width 0.2) (layer "F.Cu") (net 13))
 (segment (start 129.794 90.614) (end 130.111 90.614) (width 0.2) (layer "F.Cu") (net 13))
 (via (at 140.060765 89.174235) (size 0.6) (drill 0.3) (layers "F.Cu" "B.Cu") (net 13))
 (via (at 144.145 91.854) (size 0.6) (drill 0.3) (layers "F.Cu" "B.Cu") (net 13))
 (via (at 130.175 90.678) (size 0.6) (drill 0.3) (layers "F.Cu" "B.Cu") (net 13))
 (via (at 139.203472 90.014) (size 0.6) (drill 0.3) (layers "F.Cu" "B.Cu") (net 13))
 (segment (start 140.060765 89.174235) (end 141.465235 89.174235) (width 0.2) (layer "B.Cu") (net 13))
 (segment (start 130.175 90.678) (end 130.839 90.014) (width 0.2) (layer "B.Cu") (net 13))
 (segment (start 130.839 90.014) (end 139.203472 90.014) (width 0.2) (layer "B.Cu") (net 13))
 (segment (start 141.465235 89.174235) (end 144.145 91.854) (width 0.2) (layer "B.Cu") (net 13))
 (segment (start 146.05 99.06) (end 146.05 96.814471) (width 0.2) (layer "F.Cu") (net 1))
 (segment (start 146.05 96.814471) (end 142.24 93.004471) (width 0.2) (layer "F.Cu") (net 1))
 (segment (start 142.24 87.089) (end 141.605 86.454) (width 0.2) (layer "F.Cu") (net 1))
 (segment (start 142.24 93.004471) (end 142.24 87.089) (width 0.2) (layer "F.Cu") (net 1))
 (segment (start 140.335 85.725) (end 140.335 86.454) (width 0.2) (layer "F.Cu") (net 6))
 (segment (start 139.95 82.05659) (end 139.95 82.739) (width 0.2) (layer "F.Cu") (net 6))
 (segment (start 139.55441 81.661) (end 139.95 82.05659) (width 0.2) (layer "F.Cu") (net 6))
 (segment (start 145.041 85.404) (end 140.656 85.404) (width 0.2) (layer "F.Cu") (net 6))
 (segment (start 139.95 86.069) (end 140.335 86.454) (width 0.2) (layer "F.Cu") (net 6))
 (segment (start 146.086 86.449) (end 146.086 86.832) (width 0.2) (layer "F.Cu") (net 6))
 (segment (start 146.086 86.832) (end 146.05 86.868) (width 0.2) (layer "F.Cu") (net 6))
 (segment (start 138.95 82.739) (end 138.95 82.05659) (width 0.2) (layer "F.Cu") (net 6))
 (segment (start 146.086 86.449) (end 145.041 85.404) (width 0.2) (layer "F.Cu") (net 6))
 (segment (start 139.95 82.739) (end 139.95 86.069) (width 0.2) (layer "F.Cu") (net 6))
 (segment (start 138.95 82.05659) (end 139.34559 81.661) (width 0.2) (layer "F.Cu") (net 6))
 (segment (start 139.34559 81.661) (end 139.55441 81.661) (width 0.2) (layer "F.Cu") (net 6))
 (segment (start 140.656 85.404) (end 140.335 85.725) (width 0.2) (layer "F.Cu") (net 6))
 (via (at 146.05 86.868) (size 0.6) (drill 0.3) (layers "F.Cu" "B.Cu") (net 6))
 (via (at 146.086 94.399) (size 0.6) (drill 0.3) (layers "F.Cu" "B.Cu") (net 6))
 (segment (start 146.05 86.868) (end 146.05 94.363) (width 0.2) (layer "B.Cu") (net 6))
 (segment (start 146.05 94.363) (end 146.086 94.399) (width 0.2) (layer "B.Cu") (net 6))
 (segment (start 133.73 80.518) (end 133.604 80.392) (width 0.2) (layer "F.Cu") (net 19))
 (segment (start 137.95 81.784406) (end 136.683594 80.518) (width 0.2) (layer "F.Cu") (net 19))
 (segment (start 136.683594 80.518) (end 135.98 80.518) (width 0.2) (layer "F.Cu") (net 19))
 (segment (start 134.747 80.518) (end 133.73 80.518) (width 0.2) (layer "F.Cu") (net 19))
 (segment (start 137.95 82.739) (end 137.95 81.784406) (width 0.2) (layer "F.Cu") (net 19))
 (via (at 135.98 80.518) (size 0.6) (drill 0.3) (layers "F.Cu" "B.Cu") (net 19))
 (via (at 134.747 80.518) (size 0.6) (drill 0.3) (layers "F.Cu" "B.Cu") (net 19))
 (segment (start 135.98 80.518) (end 134.747 80.518) (width 0.2) (layer "B.Cu") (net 19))
 (segment (start 145.795 80.391) (end 145.796 80.392) (width 0.2) (layer "F.Cu") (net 17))
 (segment (start 142.61559 80.391) (end 143.42 80.391) (width 0.2) (layer "F.Cu") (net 17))
 (segment (start 144.62 80.391) (end 145.795 80.391) (width 0.2) (layer "F.Cu") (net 17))
 (segment (start 140.95 82.739) (end 140.95 82.05659) (width 0.2) (layer "F.Cu") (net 17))
 (segment (start 140.95 82.05659) (end 142.61559 80.391) (width 0.2) (layer "F.Cu") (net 17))
 (via (at 143.42 80.391) (size 0.6) (drill 0.3) (layers "F.Cu" "B.Cu") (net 17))
 (via (at 144.62 80.391) (size 0.6) (drill 0.3) (layers "F.Cu" "B.Cu") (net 17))
 (segment (start 143.42 80.391) (end 144.62 80.391) (width 0.2) (layer "B.Cu") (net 17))
 (segment (start 150.558 86.421) (end 150.586 86.449) (width 0.2) (layer "F.Cu") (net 5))
 (segment (start 150.558 84.455) (end 150.558 86.421) (width 0.2) (layer "F.Cu") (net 5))
 (segment (start 150.586 86.449) (end 150.586 86.832) (width 0.2) (layer "F.Cu") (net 5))
 (segment (start 150.586 86.832) (end 150.622 86.868) (width 0.2) (layer "F.Cu") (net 5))
 (via (at 150.622 86.868) (size 0.6) (drill 0.3) (layers "F.Cu" "B.Cu") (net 5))
 (via (at 150.586 94.399) (size 0.6) (drill 0.3) (layers "F.Cu" "B.Cu") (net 5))
 (segment (start 150.622 94.363) (end 150.586 94.399) (width 0.2) (layer "B.Cu") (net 5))
 (segment (start 150.622 86.868) (end 150.622 94.363) (width 0.2) (layer "B.Cu") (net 5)))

